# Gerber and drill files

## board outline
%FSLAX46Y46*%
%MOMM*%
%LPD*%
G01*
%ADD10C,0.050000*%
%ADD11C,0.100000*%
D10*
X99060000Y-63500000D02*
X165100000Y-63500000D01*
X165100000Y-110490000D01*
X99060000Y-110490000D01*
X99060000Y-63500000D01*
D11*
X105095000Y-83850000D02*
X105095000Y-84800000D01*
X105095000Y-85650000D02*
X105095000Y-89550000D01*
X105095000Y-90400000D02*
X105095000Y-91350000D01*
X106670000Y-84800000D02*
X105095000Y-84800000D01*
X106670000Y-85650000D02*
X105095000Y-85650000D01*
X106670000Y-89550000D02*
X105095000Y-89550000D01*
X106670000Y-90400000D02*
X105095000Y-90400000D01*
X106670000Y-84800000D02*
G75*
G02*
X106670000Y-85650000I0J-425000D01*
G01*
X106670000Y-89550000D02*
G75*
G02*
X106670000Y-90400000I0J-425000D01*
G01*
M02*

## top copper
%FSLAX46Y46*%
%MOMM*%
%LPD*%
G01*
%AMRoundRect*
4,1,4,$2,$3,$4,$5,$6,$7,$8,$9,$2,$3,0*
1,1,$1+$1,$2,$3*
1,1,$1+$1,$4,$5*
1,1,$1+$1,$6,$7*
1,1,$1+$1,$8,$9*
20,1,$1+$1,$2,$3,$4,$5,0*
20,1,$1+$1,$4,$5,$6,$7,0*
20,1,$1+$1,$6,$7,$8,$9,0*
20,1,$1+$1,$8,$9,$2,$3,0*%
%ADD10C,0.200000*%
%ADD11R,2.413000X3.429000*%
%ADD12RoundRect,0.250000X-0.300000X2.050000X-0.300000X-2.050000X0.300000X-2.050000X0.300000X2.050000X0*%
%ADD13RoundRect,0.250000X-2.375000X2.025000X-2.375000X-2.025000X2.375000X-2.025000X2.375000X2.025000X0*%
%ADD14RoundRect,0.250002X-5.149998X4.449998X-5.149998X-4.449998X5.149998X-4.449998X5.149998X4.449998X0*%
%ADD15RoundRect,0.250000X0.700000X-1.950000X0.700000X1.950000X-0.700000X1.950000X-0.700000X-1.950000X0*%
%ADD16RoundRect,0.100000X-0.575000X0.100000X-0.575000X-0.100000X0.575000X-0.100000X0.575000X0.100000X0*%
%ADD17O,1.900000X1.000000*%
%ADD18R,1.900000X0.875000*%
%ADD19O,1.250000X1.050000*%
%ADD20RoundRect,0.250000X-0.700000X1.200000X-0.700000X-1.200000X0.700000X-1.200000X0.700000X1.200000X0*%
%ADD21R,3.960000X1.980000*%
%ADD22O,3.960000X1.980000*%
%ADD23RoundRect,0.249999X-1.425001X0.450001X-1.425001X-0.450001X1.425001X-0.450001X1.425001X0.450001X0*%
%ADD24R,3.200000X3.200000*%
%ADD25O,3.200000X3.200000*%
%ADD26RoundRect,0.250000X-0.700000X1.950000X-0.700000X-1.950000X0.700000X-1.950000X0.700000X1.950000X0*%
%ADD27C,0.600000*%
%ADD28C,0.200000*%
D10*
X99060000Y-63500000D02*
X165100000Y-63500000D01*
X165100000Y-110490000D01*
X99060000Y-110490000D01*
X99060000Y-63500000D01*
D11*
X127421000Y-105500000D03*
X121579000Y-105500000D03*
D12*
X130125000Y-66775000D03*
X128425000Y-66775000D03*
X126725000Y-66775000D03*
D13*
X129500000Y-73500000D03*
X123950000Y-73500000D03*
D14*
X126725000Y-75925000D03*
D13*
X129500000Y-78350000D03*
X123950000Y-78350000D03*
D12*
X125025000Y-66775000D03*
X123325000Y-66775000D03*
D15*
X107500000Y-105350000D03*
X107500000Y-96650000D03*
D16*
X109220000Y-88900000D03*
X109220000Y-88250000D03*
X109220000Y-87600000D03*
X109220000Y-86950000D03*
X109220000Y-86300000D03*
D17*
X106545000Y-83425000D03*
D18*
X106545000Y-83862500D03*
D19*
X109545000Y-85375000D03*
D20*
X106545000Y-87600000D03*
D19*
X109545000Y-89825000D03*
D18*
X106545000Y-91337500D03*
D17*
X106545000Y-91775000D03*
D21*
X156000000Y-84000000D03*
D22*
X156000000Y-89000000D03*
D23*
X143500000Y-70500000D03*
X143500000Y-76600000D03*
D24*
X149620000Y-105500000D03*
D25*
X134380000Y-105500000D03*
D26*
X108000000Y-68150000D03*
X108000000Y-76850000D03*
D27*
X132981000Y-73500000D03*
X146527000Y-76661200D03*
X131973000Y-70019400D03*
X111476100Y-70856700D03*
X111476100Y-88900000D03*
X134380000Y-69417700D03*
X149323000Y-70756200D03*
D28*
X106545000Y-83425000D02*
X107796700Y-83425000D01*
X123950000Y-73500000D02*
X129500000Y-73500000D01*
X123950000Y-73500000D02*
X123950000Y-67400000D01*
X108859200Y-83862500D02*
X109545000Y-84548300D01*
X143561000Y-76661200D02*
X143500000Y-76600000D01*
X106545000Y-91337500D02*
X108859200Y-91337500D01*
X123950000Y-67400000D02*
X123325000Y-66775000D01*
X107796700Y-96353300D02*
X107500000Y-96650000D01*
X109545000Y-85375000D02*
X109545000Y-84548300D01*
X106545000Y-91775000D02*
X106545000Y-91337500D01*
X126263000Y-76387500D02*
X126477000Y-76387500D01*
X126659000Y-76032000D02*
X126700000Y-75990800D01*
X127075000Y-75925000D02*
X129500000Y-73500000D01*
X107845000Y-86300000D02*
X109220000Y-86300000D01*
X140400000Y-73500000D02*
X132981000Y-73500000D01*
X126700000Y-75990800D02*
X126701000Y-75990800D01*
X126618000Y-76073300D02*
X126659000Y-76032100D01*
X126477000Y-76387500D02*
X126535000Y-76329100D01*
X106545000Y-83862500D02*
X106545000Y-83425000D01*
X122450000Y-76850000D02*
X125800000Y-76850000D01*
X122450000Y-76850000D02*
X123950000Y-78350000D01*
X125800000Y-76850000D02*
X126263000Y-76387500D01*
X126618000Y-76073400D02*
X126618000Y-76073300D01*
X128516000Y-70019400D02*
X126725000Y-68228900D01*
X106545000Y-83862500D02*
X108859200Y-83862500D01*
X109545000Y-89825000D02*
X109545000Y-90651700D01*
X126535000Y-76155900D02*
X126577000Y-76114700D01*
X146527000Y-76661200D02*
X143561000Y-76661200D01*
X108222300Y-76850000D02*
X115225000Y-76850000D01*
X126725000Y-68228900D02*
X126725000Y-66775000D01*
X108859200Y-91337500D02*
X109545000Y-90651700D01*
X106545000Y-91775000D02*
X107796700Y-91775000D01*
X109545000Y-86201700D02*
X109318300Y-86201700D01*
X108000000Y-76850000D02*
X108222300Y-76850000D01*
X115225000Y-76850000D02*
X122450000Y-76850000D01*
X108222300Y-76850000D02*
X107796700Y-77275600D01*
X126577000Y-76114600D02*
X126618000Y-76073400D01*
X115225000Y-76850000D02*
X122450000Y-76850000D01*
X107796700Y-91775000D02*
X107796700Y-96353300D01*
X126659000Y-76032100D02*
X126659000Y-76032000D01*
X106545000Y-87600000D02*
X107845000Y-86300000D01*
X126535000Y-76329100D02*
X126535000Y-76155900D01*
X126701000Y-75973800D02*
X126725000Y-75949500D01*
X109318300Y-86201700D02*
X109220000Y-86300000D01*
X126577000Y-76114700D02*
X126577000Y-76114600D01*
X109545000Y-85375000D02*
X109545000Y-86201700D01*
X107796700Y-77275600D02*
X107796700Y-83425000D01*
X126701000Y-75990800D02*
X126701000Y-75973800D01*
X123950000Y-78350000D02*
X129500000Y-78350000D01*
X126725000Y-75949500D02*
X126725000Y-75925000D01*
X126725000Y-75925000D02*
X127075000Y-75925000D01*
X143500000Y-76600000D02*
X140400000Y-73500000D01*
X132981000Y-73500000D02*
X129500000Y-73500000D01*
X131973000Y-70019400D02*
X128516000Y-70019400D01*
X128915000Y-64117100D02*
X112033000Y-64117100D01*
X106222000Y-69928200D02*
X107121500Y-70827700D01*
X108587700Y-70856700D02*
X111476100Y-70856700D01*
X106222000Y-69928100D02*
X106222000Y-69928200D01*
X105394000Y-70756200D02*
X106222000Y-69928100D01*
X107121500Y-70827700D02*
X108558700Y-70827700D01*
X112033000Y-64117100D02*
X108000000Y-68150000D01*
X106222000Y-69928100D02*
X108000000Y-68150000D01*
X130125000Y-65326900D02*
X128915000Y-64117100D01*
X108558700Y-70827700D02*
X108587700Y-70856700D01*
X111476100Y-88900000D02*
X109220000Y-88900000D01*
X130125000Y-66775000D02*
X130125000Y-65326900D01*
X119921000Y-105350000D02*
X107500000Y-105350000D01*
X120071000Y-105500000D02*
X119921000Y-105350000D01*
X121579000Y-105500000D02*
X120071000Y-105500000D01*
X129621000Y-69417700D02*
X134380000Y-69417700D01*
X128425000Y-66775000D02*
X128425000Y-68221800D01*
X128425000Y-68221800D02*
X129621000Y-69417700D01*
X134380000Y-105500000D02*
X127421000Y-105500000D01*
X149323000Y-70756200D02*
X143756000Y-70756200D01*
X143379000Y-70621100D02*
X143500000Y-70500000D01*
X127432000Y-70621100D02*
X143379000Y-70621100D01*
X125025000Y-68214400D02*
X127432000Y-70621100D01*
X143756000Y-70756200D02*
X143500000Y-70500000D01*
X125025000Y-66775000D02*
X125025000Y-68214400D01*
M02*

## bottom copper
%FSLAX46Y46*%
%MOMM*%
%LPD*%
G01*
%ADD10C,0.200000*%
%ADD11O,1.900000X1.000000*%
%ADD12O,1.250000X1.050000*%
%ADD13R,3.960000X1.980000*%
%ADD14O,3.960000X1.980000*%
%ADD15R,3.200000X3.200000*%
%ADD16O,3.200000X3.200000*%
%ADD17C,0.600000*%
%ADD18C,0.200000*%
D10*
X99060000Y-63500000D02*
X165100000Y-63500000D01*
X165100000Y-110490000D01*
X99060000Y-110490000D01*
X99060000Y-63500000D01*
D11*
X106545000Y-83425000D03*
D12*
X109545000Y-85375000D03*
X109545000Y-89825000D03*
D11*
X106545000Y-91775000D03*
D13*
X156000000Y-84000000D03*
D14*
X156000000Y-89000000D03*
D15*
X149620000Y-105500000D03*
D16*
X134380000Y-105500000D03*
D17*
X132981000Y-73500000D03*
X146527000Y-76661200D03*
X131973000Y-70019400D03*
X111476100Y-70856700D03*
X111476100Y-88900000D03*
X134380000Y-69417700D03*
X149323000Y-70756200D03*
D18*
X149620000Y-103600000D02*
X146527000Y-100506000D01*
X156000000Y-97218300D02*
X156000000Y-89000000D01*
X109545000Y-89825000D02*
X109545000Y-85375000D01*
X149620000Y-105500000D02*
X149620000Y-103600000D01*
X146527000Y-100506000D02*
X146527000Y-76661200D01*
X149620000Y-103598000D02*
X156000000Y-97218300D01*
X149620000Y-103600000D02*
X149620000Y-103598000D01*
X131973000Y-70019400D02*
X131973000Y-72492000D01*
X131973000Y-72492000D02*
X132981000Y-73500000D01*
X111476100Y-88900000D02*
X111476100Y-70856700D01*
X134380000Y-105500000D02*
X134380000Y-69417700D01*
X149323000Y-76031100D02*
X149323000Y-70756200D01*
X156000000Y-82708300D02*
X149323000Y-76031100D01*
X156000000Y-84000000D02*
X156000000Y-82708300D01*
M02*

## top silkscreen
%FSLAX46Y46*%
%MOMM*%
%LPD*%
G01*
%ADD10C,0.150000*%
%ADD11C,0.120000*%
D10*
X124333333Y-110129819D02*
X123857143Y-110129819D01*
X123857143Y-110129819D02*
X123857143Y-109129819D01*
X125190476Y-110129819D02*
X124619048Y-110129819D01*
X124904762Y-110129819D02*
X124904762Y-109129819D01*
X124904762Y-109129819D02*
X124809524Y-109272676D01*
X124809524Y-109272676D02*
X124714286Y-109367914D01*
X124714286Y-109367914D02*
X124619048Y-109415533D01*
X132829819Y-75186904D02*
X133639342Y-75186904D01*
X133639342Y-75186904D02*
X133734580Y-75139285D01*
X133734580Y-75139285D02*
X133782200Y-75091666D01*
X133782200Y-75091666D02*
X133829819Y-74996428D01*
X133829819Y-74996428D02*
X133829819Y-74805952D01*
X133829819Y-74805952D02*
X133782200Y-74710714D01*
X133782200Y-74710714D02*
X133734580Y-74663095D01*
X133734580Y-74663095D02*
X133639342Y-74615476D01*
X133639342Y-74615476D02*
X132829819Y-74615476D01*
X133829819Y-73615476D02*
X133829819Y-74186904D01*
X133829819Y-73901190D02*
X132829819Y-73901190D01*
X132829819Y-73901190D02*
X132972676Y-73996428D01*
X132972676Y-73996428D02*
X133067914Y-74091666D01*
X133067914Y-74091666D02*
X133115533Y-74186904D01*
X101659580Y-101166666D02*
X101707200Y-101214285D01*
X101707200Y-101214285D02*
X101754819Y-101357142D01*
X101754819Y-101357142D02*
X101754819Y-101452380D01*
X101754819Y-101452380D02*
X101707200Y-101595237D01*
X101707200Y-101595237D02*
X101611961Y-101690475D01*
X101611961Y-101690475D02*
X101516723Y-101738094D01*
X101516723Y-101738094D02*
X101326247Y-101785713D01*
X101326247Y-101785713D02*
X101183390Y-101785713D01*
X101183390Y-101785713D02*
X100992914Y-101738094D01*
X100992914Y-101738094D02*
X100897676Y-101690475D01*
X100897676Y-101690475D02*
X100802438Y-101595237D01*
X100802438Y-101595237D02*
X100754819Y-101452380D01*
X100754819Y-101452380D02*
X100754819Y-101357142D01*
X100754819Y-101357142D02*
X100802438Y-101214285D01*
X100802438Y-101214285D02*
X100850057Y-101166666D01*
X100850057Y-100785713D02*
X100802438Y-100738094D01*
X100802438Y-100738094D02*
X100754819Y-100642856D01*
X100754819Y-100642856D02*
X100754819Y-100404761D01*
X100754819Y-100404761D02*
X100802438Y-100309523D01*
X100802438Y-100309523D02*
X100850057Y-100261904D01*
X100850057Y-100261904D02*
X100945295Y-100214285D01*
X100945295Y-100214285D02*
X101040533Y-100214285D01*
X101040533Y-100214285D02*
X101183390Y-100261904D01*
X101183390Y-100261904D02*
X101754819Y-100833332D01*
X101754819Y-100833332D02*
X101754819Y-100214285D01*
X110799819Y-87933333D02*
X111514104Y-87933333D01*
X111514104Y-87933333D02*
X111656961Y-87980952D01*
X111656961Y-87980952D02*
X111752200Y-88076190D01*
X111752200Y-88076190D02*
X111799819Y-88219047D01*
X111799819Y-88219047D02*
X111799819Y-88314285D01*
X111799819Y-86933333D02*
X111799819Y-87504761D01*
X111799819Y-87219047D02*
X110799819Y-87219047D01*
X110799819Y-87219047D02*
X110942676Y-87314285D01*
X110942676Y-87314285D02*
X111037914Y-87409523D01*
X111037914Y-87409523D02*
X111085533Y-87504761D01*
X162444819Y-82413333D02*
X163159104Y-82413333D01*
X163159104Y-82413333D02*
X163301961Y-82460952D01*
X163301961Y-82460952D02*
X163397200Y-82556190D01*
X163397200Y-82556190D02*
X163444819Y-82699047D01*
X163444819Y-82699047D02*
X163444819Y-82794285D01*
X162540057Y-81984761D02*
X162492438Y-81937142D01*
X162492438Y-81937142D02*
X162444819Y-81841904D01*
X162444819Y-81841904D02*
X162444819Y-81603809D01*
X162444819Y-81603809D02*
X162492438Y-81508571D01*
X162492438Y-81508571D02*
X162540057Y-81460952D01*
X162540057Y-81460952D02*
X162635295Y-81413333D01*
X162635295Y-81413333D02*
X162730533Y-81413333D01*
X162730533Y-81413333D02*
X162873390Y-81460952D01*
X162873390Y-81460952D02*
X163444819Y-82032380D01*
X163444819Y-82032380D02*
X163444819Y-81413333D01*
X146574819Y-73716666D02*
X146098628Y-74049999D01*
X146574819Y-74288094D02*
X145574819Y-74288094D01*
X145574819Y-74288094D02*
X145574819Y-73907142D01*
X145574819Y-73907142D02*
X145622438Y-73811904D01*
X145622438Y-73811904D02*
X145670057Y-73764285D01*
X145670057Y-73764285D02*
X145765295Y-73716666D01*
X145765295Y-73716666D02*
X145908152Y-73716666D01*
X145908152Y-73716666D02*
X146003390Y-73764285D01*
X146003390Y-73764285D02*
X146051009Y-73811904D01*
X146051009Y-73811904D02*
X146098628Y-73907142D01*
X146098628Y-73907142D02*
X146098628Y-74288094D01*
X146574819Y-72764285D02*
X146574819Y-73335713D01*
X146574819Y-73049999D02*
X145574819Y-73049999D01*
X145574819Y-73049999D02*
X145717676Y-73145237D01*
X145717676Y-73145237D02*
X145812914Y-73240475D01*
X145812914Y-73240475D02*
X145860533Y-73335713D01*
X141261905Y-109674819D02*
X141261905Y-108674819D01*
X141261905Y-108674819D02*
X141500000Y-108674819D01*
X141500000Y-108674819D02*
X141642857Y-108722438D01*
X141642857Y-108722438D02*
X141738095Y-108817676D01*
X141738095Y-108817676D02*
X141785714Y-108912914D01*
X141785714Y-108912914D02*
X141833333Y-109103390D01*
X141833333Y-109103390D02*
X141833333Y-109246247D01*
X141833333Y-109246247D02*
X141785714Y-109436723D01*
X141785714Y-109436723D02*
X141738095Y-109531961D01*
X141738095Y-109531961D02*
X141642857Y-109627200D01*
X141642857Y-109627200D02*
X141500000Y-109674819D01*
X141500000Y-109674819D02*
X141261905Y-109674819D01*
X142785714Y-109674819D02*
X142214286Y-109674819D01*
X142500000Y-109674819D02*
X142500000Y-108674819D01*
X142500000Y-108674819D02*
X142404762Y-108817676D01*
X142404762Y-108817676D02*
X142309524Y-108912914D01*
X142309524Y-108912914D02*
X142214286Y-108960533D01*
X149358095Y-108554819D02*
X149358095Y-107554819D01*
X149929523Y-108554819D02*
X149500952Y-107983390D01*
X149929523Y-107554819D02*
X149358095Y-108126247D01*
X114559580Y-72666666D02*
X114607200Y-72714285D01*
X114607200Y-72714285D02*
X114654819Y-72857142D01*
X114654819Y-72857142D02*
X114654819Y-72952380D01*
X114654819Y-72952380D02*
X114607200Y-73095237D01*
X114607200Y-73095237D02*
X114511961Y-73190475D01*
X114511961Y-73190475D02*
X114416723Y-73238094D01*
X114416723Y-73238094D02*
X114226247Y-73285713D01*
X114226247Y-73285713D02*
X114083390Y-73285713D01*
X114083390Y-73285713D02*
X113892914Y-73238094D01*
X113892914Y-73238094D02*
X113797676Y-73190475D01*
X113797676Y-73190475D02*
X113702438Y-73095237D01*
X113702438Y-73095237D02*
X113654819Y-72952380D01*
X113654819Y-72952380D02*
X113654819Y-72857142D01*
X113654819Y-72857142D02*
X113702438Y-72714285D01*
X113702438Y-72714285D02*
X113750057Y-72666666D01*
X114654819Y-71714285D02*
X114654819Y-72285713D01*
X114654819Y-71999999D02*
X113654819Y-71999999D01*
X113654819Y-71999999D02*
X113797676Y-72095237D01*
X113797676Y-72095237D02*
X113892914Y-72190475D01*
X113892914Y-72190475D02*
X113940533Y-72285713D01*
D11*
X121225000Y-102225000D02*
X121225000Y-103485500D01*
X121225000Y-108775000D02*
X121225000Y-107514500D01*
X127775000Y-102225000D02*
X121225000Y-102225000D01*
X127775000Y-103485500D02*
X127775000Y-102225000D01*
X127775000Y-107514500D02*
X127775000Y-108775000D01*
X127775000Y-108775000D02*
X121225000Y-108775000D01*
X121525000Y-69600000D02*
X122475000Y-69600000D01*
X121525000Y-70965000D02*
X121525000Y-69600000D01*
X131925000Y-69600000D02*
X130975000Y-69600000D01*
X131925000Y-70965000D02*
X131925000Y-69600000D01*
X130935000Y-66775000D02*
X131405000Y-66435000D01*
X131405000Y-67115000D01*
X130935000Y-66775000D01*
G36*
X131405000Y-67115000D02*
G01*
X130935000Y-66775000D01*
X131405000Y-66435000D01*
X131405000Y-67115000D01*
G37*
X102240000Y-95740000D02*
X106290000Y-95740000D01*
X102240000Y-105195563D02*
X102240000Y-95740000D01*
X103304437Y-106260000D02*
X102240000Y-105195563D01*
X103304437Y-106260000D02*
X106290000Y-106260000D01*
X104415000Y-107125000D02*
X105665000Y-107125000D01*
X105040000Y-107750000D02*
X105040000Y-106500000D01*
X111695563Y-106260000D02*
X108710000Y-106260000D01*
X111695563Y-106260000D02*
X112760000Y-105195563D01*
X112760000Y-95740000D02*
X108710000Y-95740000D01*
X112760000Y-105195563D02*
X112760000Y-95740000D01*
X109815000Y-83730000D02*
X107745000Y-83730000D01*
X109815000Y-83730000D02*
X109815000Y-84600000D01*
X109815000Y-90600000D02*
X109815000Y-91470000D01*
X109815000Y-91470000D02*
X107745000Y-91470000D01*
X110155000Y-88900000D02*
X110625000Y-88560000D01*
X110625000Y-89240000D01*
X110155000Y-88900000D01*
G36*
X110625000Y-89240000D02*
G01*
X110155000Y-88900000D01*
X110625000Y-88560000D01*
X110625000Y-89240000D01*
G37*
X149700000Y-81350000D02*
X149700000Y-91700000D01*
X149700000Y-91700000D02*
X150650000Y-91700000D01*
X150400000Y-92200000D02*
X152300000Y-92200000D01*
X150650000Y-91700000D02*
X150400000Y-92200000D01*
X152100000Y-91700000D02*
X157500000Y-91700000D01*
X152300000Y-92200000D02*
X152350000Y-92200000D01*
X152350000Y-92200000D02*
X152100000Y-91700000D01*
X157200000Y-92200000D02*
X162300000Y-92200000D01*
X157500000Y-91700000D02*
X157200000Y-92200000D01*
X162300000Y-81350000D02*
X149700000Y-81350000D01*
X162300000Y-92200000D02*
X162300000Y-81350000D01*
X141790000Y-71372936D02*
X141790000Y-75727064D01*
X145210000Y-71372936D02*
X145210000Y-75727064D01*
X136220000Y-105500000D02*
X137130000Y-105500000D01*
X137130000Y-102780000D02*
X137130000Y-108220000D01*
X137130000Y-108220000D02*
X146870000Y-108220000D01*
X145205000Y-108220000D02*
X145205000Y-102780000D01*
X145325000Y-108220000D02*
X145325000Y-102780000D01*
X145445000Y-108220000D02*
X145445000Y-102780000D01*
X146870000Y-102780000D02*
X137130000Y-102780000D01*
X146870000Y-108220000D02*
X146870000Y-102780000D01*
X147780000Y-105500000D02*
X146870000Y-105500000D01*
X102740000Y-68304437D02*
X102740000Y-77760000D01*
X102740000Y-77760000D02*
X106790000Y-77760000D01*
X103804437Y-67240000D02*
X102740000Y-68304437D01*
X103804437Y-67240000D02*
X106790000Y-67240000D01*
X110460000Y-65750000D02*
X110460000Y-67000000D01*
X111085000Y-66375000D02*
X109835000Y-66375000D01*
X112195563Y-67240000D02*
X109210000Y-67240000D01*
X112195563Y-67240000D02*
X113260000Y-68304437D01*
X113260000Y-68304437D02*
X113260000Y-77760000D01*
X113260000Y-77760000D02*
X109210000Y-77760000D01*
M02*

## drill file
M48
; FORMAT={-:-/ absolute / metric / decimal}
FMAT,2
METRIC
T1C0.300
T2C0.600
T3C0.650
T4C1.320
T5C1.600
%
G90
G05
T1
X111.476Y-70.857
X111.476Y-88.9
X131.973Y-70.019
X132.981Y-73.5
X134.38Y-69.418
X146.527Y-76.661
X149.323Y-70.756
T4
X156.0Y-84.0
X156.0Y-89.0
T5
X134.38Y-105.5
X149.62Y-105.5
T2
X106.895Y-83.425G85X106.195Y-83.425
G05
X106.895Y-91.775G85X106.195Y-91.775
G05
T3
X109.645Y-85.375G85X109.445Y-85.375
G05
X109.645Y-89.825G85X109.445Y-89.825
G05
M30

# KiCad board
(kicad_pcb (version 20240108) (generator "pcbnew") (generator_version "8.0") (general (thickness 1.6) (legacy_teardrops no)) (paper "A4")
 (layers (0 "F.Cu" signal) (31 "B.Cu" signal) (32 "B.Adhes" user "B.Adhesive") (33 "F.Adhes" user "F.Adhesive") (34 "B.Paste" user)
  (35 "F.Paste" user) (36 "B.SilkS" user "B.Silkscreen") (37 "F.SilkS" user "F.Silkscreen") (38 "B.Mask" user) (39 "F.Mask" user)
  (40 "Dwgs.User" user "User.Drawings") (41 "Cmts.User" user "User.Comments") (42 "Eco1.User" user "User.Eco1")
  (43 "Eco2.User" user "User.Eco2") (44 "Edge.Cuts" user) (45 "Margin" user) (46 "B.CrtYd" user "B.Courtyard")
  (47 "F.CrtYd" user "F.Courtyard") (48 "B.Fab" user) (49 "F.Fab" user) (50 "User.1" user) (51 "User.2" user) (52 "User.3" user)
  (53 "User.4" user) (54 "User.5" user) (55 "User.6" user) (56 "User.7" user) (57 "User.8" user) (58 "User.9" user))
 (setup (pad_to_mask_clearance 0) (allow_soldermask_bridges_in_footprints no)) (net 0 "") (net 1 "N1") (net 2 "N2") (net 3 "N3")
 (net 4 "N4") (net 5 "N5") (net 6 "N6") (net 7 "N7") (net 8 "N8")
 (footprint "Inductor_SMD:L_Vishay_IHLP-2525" (layer "F.Cu") (at 124.5 105.5 180)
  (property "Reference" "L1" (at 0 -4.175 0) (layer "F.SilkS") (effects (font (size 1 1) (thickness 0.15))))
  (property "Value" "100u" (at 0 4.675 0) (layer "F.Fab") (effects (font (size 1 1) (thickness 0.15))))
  (fp_line (start 3.275 3.275) (end 3.275 2.0145) (stroke (width 0.12) (type solid)) (layer "F.SilkS"))
  (fp_line (start 3.275 -3.275) (end 3.275 -2.0145) (stroke (width 0.12) (type solid)) (layer "F.SilkS"))
  (fp_line (start -3.275 3.275) (end 3.275 3.275) (stroke (width 0.12) (type solid)) (layer "F.SilkS"))
  (fp_line (start -3.275 2.0145) (end -3.275 3.275) (stroke (width 0.12) (type solid)) (layer "F.SilkS"))
  (fp_line (start -3.275 -2.0145) (end -3.275 -3.275) (stroke (width 0.12) (type solid)) (layer "F.SilkS"))
  (fp_line (start -3.275 -3.275) (end 3.275 -3.275) (stroke (width 0.12) (type solid)) (layer "F.SilkS"))
  (pad "1" smd rect (at -2.921 0 180) (size 2.413 3.429) (layers "F.Cu" "F.Paste" "F.Mask") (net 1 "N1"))
  (pad "2" smd rect (at 2.921 0 180) (size 2.413 3.429) (layers "F.Cu" "F.Paste" "F.Mask") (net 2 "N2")))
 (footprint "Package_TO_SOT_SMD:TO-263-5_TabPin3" (layer "F.Cu") (at 126.725 74.425 -90)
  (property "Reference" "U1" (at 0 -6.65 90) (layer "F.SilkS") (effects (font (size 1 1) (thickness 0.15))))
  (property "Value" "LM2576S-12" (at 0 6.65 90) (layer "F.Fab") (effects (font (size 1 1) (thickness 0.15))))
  (fp_line (start -4.825 5.2) (end -4.825 4.25) (stroke (width 0.12) (type solid)) (layer "F.SilkS"))
  (fp_line (start -3.46 5.2) (end -4.825 5.2) (stroke (width 0.12) (type solid)) (layer "F.SilkS"))
  (fp_line (start -4.825 -5.2) (end -4.825 -4.25) (stroke (width 0.12) (type solid)) (layer "F.SilkS"))
  (fp_line (start -3.46 -5.2) (end -4.825 -5.2) (stroke (width 0.12) (type solid)) (layer "F.SilkS"))
  (fp_poly
   (pts (xy -7.65 -4.21) (xy -7.99 -4.68) (xy -7.31 -4.68) (xy -7.65 -4.21)) (stroke (width 0.12) (type solid)) (fill solid)
   (layer "F.SilkS"))
  (pad "1" smd roundrect (at -7.65 -3.4 270) (size 4.6 1.1) (layers "F.Cu" "F.Paste" "F.Mask") (roundrect_rratio 0.227273) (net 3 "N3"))
  (pad "2" smd roundrect (at -7.65 -1.7 270) (size 4.6 1.1) (layers "F.Cu" "F.Paste" "F.Mask") (roundrect_rratio 0.227273) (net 1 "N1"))
  (pad "3" smd roundrect (at -7.65 0 270) (size 4.6 1.1) (layers "F.Cu" "F.Paste" "F.Mask") (roundrect_rratio 0.227273) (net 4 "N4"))
  (pad "3" smd roundrect (at -0.925 -2.775 270) (size 4.55 5.25) (layers "F.Cu" "F.Paste") (roundrect_rratio 0.054945) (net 4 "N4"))
  (pad "3" smd roundrect (at -0.925 2.775 270) (size 4.55 5.25) (layers "F.Cu" "F.Paste") (roundrect_rratio 0.054945) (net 4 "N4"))
  (pad "3" smd roundrect (at 1.5 0 270) (size 9.4 10.8) (layers "F.Cu" "F.Mask") (roundrect_rratio 0.026596) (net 4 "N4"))
  (pad "3" smd roundrect (at 3.925 -2.775 270) (size 4.55 5.25) (layers "F.Cu" "F.Paste") (roundrect_rratio 0.054945) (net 4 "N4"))
  (pad "3" smd roundrect (at 3.925 2.775 270) (size 4.55 5.25) (layers "F.Cu" "F.Paste") (roundrect_rratio 0.054945) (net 4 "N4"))
  (pad "4" smd roundrect (at -7.65 1.7 270) (size 4.6 1.1) (layers "F.Cu" "F.Paste" "F.Mask") (roundrect_rratio 0.227273) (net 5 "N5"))
  (pad "5" smd roundrect (at -7.65 3.4 270) (size 4.6 1.1) (layers "F.Cu" "F.Paste" "F.Mask") (roundrect_rratio 0.227273) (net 4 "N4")))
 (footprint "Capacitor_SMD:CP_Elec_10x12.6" (layer "F.Cu") (at 107.5 101 90)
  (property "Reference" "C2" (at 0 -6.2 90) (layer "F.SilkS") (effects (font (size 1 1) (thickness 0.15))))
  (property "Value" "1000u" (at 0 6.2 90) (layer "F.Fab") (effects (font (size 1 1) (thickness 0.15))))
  (fp_line (start 5.26 -5.26) (end 5.26 -1.21) (stroke (width 0.12) (type solid)) (layer "F.SilkS"))
  (fp_line (start -4.195563 -5.26) (end 5.26 -5.26) (stroke (width 0.12) (type solid)) (layer "F.SilkS"))
  (fp_line (start -5.26 -4.195563) (end -4.195563 -5.26) (stroke (width 0.12) (type solid)) (layer "F.SilkS"))
  (fp_line (start -5.26 -4.195563) (end -5.26 -1.21) (stroke (width 0.12) (type solid)) (layer "F.SilkS"))
  (fp_line (start -6.125 -3.085) (end -6.125 -1.835) (stroke (width 0.12) (type solid)) (layer "F.SilkS"))
  (fp_line (start -6.75 -2.46) (end -5.5 -2.46) (stroke (width 0.12) (type solid)) (layer "F.SilkS"))
  (fp_line (start -5.26 4.195563) (end -5.26 1.21) (stroke (width 0.12) (type solid)) (layer "F.SilkS"))
  (fp_line (start -5.26 4.195563) (end -4.195563 5.26) (stroke (width 0.12) (type solid)) (layer "F.SilkS"))
  (fp_line (start 5.26 5.26) (end 5.26 1.21) (stroke (width 0.12) (type solid)) (layer "F.SilkS"))
  (fp_line (start -4.195563 5.26) (end 5.26 5.26) (stroke (width 0.12) (type solid)) (layer "F.SilkS"))
  (pad "1" smd roundrect (at -4.35 0 90) (size 4.4 1.9) (layers "F.Cu" "F.Paste" "F.Mask") (roundrect_rratio 0.131579) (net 2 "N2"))
  (pad "2" smd roundrect (at 4.35 0 90) (size 4.4 1.9) (layers "F.Cu" "F.Paste" "F.Mask") (roundrect_rratio 0.131579) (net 4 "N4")))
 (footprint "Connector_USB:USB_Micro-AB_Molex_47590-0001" (layer "F.Cu") (at 106.195 87.6 -90)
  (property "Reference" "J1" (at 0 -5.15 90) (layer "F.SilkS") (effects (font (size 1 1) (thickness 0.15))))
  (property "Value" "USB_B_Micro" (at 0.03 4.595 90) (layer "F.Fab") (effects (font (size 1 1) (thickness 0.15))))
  (fp_line (start -3.87 -3.62) (end -3.87 -1.55) (stroke (width 0.12) (type solid)) (layer "F.SilkS"))
  (fp_line (start -3.87 -3.62) (end -3 -3.62) (stroke (width 0.12) (type solid)) (layer "F.SilkS"))
  (fp_line (start 3 -3.62) (end 3.87 -3.62) (stroke (width 0.12) (type solid)) (layer "F.SilkS"))
  (fp_line (start 3.87 -3.62) (end 3.87 -1.55) (stroke (width 0.12) (type solid)) (layer "F.SilkS"))
  (fp_poly
   (pts (xy 1.3 -3.96) (xy 0.96 -4.43) (xy 1.64 -4.43) (xy 1.3 -3.96)) (stroke (width 0.12) (type solid)) (fill solid) (layer "F.SilkS"))
  (fp_line (start -3.75 1.1) (end -2.8 1.1) (stroke (width 0.1) (type solid)) (layer "Edge.Cuts"))
  (fp_line (start -1.95 1.1) (end 1.95 1.1) (stroke (width 0.1) (type solid)) (layer "Edge.Cuts"))
  (fp_line (start 2.8 1.1) (end 3.75 1.1) (stroke (width 0.1) (type solid)) (layer "Edge.Cuts"))
  (fp_line (start -2.8 -0.475) (end -2.8 1.1) (stroke (width 0.1) (type solid)) (layer "Edge.Cuts"))
  (fp_line (start -1.95 -0.475) (end -1.95 1.1) (stroke (width 0.1) (type solid)) (layer "Edge.Cuts"))
  (fp_line (start 1.95 -0.475) (end 1.95 1.1) (stroke (width 0.1) (type solid)) (layer "Edge.Cuts"))
  (fp_line (start 2.8 -0.475) (end 2.8 1.1) (stroke (width 0.1) (type solid)) (layer "Edge.Cuts"))
  (fp_arc (start -2.8 -0.475) (mid -2.375 -0.9) (end -1.95 -0.475) (stroke (width 0.1) (type solid)) (layer "Edge.Cuts"))
  (fp_arc (start 1.95 -0.475) (mid 2.375 -0.9) (end 2.8 -0.475) (stroke (width 0.1) (type solid)) (layer "Edge.Cuts"))
  (pad "" smd rect (at -3.5 -0.35 270) (size 0.3 0.85) (layers "F.Paste"))
  (pad "" smd rect (at 3.5 -0.35 270) (size 0.3 0.85) (layers "F.Paste"))
  (pad "1" smd roundrect (at 1.3 -3.025 270) (size 0.4 1.35) (layers "F.Cu" "F.Paste" "F.Mask") (roundrect_rratio 0.25) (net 3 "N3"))
  (pad "2" smd roundrect (at 0.65 -3.025 270) (size 0.4 1.35) (layers "F.Cu" "F.Paste" "F.Mask") (roundrect_rratio 0.25) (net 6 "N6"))
  (pad "3" smd roundrect (at 0 -3.025 270) (size 0.4 1.35) (layers "F.Cu" "F.Paste" "F.Mask") (roundrect_rratio 0.25) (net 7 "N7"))
  (pad "4" smd roundrect (at -0.65 -3.025 270) (size 0.4 1.35) (layers "F.Cu" "F.Paste" "F.Mask") (roundrect_rratio 0.25) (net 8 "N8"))
  (pad "5" smd roundrect (at -1.3 -3.025 270) (size 0.4 1.35) (layers "F.Cu" "F.Paste" "F.Mask") (roundrect_rratio 0.25) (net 4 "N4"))
  (pad "6" thru_hole oval (at -4.175 -0.35 270) (size 1 1.9) (drill oval 0.6 1.3) (layers "*.Cu" "*.Mask") (remove_unused_layers no)
   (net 4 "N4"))
  (pad "6" smd rect (at -3.7375 -0.35 270) (size 0.875 1.9) (layers "F.Cu" "F.Mask") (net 4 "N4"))
  (pad "6" thru_hole oval (at -2.225 -3.35 270) (size 1.05 1.25) (drill oval 0.65 0.85) (layers "*.Cu" "*.Mask") (remove_unused_layers no)
   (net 4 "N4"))
  (pad "6" smd roundrect (at 0 -0.35 270) (size 2.9 1.9) (layers "F.Cu" "F.Paste" "F.Mask") (roundrect_rratio 0.1315789474) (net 4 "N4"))
  (pad "6" thru_hole oval (at 2.225 -3.35 270) (size 1.05 1.25) (drill oval 0.65 0.85) (layers "*.Cu" "*.Mask") (remove_unused_layers no)
   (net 4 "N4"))
  (pad "6" smd rect (at 3.7375 -0.35 270) (size 0.875 1.9) (layers "F.Cu" "F.Mask") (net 4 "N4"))
  (pad "6" thru_hole oval (at 4.175 -0.35 270) (size 1 1.9) (drill oval 0.6 1.3) (layers "*.Cu" "*.Mask") (remove_unused_layers no)
   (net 4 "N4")))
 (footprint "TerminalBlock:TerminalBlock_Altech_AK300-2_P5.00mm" (layer "F.Cu") (at 156 84 -90)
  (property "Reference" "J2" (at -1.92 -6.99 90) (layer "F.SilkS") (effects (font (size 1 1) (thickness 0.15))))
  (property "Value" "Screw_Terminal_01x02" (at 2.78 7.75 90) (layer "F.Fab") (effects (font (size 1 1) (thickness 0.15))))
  (fp_line (start -2.65 6.3) (end 7.7 6.3) (stroke (width 0.12) (type solid)) (layer "F.SilkS"))
  (fp_line (start 7.7 6.3) (end 7.7 5.35) (stroke (width 0.12) (type solid)) (layer "F.SilkS"))
  (fp_line (start 8.2 5.6) (end 8.2 3.7) (stroke (width 0.12) (type solid)) (layer "F.SilkS"))
  (fp_line (start 7.7 5.35) (end 8.2 5.6) (stroke (width 0.12) (type solid)) (layer "F.SilkS"))
  (fp_line (start 7.7 3.9) (end 7.7 -1.5) (stroke (width 0.12) (type solid)) (layer "F.SilkS"))
  (fp_line (start 8.2 3.7) (end 8.2 3.65) (stroke (width 0.12) (type solid)) (layer "F.SilkS"))
  (fp_line (start 8.2 3.65) (end 7.7 3.9) (stroke (width 0.12) (type solid)) (layer "F.SilkS"))
  (fp_line (start 8.2 -1.2) (end 8.2 -6.3) (stroke (width 0.12) (type solid)) (layer "F.SilkS"))
  (fp_line (start 7.7 -1.5) (end 8.2 -1.2) (stroke (width 0.12) (type solid)) (layer "F.SilkS"))
  (fp_line (start -2.65 -6.3) (end -2.65 6.3) (stroke (width 0.12) (type solid)) (layer "F.SilkS"))
  (fp_line (start 8.2 -6.3) (end -2.65 -6.3) (stroke (width 0.12) (type solid)) (layer "F.SilkS"))
  (pad "1" thru_hole rect (at 0 0 270) (size 1.98 3.96) (drill 1.32) (layers "*.Cu" "*.Mask") (remove_unused_layers no) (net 5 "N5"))
  (pad "2" thru_hole oval (at 5 0 270) (size 1.98 3.96) (drill 1.32) (layers "*.Cu" "*.Mask") (remove_unused_layers no) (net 4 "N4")))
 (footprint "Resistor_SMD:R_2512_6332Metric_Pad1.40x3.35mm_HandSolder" (layer "F.Cu") (at 143.5 73.55 -90)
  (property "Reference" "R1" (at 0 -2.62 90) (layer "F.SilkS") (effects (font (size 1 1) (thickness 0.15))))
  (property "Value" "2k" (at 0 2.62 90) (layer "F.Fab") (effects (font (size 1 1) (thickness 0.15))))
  (fp_line (start -2.177064 1.71) (end 2.177064 1.71) (stroke (width 0.12) (type solid)) (layer "F.SilkS"))
  (fp_line (start -2.177064 -1.71) (end 2.177064 -1.71) (stroke (width 0.12) (type solid)) (layer "F.SilkS"))
  (pad "1" smd roundrect (at -3.05 0 270) (size 1.4 3.35) (layers "F.Cu" "F.Paste" "F.Mask") (roundrect_rratio 0.178571) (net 5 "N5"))
  (pad "2" smd roundrect (at 3.05 0 270) (size 1.4 3.35) (layers "F.Cu" "F.Paste" "F.Mask") (roundrect_rratio 0.178571) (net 4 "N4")))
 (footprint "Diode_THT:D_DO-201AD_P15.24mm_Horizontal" (layer "F.Cu") (at 149.62 105.5 180)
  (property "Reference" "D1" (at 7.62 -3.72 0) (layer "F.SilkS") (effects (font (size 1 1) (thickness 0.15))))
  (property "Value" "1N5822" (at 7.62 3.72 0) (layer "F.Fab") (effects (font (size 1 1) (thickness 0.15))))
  (fp_line (start 13.4 0) (end 12.49 0) (stroke (width 0.12) (type solid)) (layer "F.SilkS"))
  (fp_line (start 12.49 2.72) (end 12.49 -2.72) (stroke (width 0.12) (type solid)) (layer "F.SilkS"))
  (fp_line (start 12.49 -2.72) (end 2.75 -2.72) (stroke (width 0.12) (type solid)) (layer "F.SilkS"))
  (fp_line (start 4.415 -2.72) (end 4.415 2.72) (stroke (width 0.12) (type solid)) (layer "F.SilkS"))
  (fp_line (start 4.295 -2.72) (end 4.295 2.72) (stroke (width 0.12) (type solid)) (layer "F.SilkS"))
  (fp_line (start 4.175 -2.72) (end 4.175 2.72) (stroke (width 0.12) (type solid)) (layer "F.SilkS"))
  (fp_line (start 2.75 2.72) (end 12.49 2.72) (stroke (width 0.12) (type solid)) (layer "F.SilkS"))
  (fp_line (start 2.75 -2.72) (end 2.75 2.72) (stroke (width 0.12) (type solid)) (layer "F.SilkS"))
  (fp_line (start 1.84 0) (end 2.75 0) (stroke (width 0.12) (type solid)) (layer "F.SilkS"))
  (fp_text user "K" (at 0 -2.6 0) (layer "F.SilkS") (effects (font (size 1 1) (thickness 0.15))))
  (pad "1" thru_hole rect (at 0 0 180) (size 3.2 3.2) (drill 1.6) (layers "*.Cu" "*.Mask") (remove_unused_layers no) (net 4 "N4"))
  (pad "2" thru_hole oval (at 15.24 0 180) (size 3.2 3.2) (drill 1.6) (layers "*.Cu" "*.Mask") (remove_unused_layers no) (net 1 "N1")))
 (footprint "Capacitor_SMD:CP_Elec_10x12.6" (layer "F.Cu") (at 108 72.5 -90)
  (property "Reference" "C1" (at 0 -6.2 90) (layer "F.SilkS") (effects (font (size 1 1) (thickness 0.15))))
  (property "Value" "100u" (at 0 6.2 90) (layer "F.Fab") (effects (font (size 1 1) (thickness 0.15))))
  (fp_line (start -4.195563 5.26) (end 5.26 5.26) (stroke (width 0.12) (type solid)) (layer "F.SilkS"))
  (fp_line (start 5.26 5.26) (end 5.26 1.21) (stroke (width 0.12) (type solid)) (layer "F.SilkS"))
  (fp_line (start -5.26 4.195563) (end -4.195563 5.26) (stroke (width 0.12) (type solid)) (layer "F.SilkS"))
  (fp_line (start -5.26 4.195563) (end -5.26 1.21) (stroke (width 0.12) (type solid)) (layer "F.SilkS"))
  (fp_line (start -6.75 -2.46) (end -5.5 -2.46) (stroke (width 0.12) (type solid)) (layer "F.SilkS"))
  (fp_line (start -6.125 -3.085) (end -6.125 -1.835) (stroke (width 0.12) (type solid)) (layer "F.SilkS"))
  (fp_line (start -5.26 -4.195563) (end -5.26 -1.21) (stroke (width 0.12) (type solid)) (layer "F.SilkS"))
  (fp_line (start -5.26 -4.195563) (end -4.195563 -5.26) (stroke (width 0.12) (type solid)) (layer "F.SilkS"))
  (fp_line (start -4.195563 -5.26) (end 5.26 -5.26) (stroke (width 0.12) (type solid)) (layer "F.SilkS"))
  (fp_line (start 5.26 -5.26) (end 5.26 -1.21) (stroke (width 0.12) (type solid)) (layer "F.SilkS"))
  (pad "1" smd roundrect (at -4.35 0 270) (size 4.4 1.9) (layers "F.Cu" "F.Paste" "F.Mask") (roundrect_rratio 0.131579) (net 3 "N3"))
  (pad "2" smd roundrect (at 4.35 0 270) (size 4.4 1.9) (layers "F.Cu" "F.Paste" "F.Mask") (roundrect_rratio 0.131579) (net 4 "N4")))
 (gr_rect (start 99.06 63.5) (end 165.1 110.49) (stroke (width 0.2) (type default)) (fill none) (layer "F.Cu"))
 (gr_rect (start 99.06 63.5) (end 165.1 110.49) (stroke (width 0.2) (type default)) (fill none) (layer "B.Cu"))
 (gr_rect (start 99.06 63.5) (end 165.1 110.49) (stroke (width 0.05) (type default)) (fill none) (layer "Edge.Cuts"))
 (segment (start 106.545 83.425) (end 107.7967 83.425) (width 0.2) (layer "F.Cu") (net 4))
 (segment (start 123.95 73.5) (end 129.5 73.5) (width 0.2) (layer "F.Cu") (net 4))
 (segment (start 123.95 73.5) (end 123.95 67.4) (width 0.2) (layer "F.Cu") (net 4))
 (segment (start 108.8592 83.8625) (end 109.545 84.5483) (width 0.2) (layer "F.Cu") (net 4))
 (segment (start 143.561 76.6612) (end 143.5 76.6) (width 0.2) (layer "F.Cu") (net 4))
 (segment (start 106.545 91.3375) (end 108.8592 91.3375) (width 0.2) (layer "F.Cu") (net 4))
 (segment (start 123.95 67.4) (end 123.325 66.775) (width 0.2) (layer "F.Cu") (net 4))
 (segment (start 107.7967 96.3533) (end 107.5 96.65) (width 0.2) (layer "F.Cu") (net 4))
 (segment (start 109.545 85.375) (end 109.545 84.5483) (width 0.2) (layer "F.Cu") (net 4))
 (segment (start 106.545 91.775) (end 106.545 91.3375) (width 0.2) (layer "F.Cu") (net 4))
 (segment (start 126.263 76.3875) (end 126.477 76.3875) (width 0.2) (layer "F.Cu") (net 4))
 (segment (start 126.659 76.032) (end 126.7 75.9908) (width 0.2) (layer "F.Cu") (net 4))
 (segment (start 127.075 75.925) (end 129.5 73.5) (width 0.2) (layer "F.Cu") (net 4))
 (segment (start 107.845 86.3) (end 109.22 86.3) (width 0.2) (layer "F.Cu") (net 4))
 (segment (start 140.4 73.5) (end 132.981 73.5) (width 0.2) (layer "F.Cu") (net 4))
 (segment (start 126.7 75.9908) (end 126.701 75.9908) (width 0.2) (layer "F.Cu") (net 4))
 (segment (start 126.618 76.0733) (end 126.659 76.0321) (width 0.2) (layer "F.Cu") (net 4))
 (segment (start 126.477 76.3875) (end 126.535 76.3291) (width 0.2) (layer "F.Cu") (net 4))
 (segment (start 106.545 83.8625) (end 106.545 83.425) (width 0.2) (layer "F.Cu") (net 4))
 (segment (start 122.45 76.85) (end 125.8 76.85) (width 0.2) (layer "F.Cu") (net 4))
 (segment (start 122.45 76.85) (end 123.95 78.35) (width 0.2) (layer "F.Cu") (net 4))
 (segment (start 125.8 76.85) (end 126.263 76.3875) (width 0.2) (layer "F.Cu") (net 4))
 (segment (start 126.618 76.0734) (end 126.618 76.0733) (width 0.2) (layer "F.Cu") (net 4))
 (segment (start 128.516 70.0194) (end 126.725 68.2289) (width 0.2) (layer "F.Cu") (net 4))
 (segment (start 106.545 83.8625) (end 108.8592 83.8625) (width 0.2) (layer "F.Cu") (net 4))
 (segment (start 109.545 89.825) (end 109.545 90.6517) (width 0.2) (layer "F.Cu") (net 4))
 (segment (start 126.535 76.1559) (end 126.577 76.1147) (width 0.2) (layer "F.Cu") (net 4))
 (segment (start 146.527 76.6612) (end 143.561 76.6612) (width 0.2) (layer "F.Cu") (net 4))
 (segment (start 108.2223 76.85) (end 115.225 76.85) (width 0.2) (layer "F.Cu") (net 4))
 (segment (start 126.725 68.2289) (end 126.725 66.775) (width 0.2) (layer "F.Cu") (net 4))
 (segment (start 108.8592 91.3375) (end 109.545 90.6517) (width 0.2) (layer "F.Cu") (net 4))
 (segment (start 106.545 91.775) (end 107.7967 91.775) (width 0.2) (layer "F.Cu") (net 4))
 (segment (start 109.545 86.2017) (end 109.3183 86.2017) (width 0.2) (layer "F.Cu") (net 4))
 (segment (start 108 76.85) (end 108.2223 76.85) (width 0.2) (layer "F.Cu") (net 4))
 (segment (start 115.225 76.85) (end 122.45 76.85) (width 0.2) (layer "F.Cu") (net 4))
 (segment (start 108.2223 76.85) (end 107.7967 77.2756) (width 0.2) (layer "F.Cu") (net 4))
 (segment (start 126.577 76.1146) (end 126.618 76.0734) (width 0.2) (layer "F.Cu") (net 4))
 (segment (start 115.225 76.85) (end 122.45 76.85) (width 0.2) (layer "F.Cu") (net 4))
 (segment (start 107.7967 91.775) (end 107.7967 96.3533) (width 0.2) (layer "F.Cu") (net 4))
 (segment (start 126.659 76.0321) (end 126.659 76.032) (width 0.2) (layer "F.Cu") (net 4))
 (segment (start 106.545 87.6) (end 107.845 86.3) (width 0.2) (layer "F.Cu") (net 4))
 (segment (start 126.535 76.3291) (end 126.535 76.1559) (width 0.2) (layer "F.Cu") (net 4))
 (segment (start 126.701 75.9738) (end 126.725 75.9495) (width 0.2) (layer "F.Cu") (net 4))
 (segment (start 109.3183 86.2017) (end 109.22 86.3) (width 0.2) (layer "F.Cu") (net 4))
 (segment (start 126.577 76.1147) (end 126.577 76.1146) (width 0.2) (layer "F.Cu") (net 4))
 (segment (start 109.545 85.375) (end 109.545 86.2017) (width 0.2) (layer "F.Cu") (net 4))
 (segment (start 107.7967 77.2756) (end 107.7967 83.425) (width 0.2) (layer "F.Cu") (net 4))
 (segment (start 126.701 75.9908) (end 126.701 75.9738) (width 0.2) (layer "F.Cu") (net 4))
 (segment (start 123.95 78.35) (end 129.5 78.35) (width 0.2) (layer "F.Cu") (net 4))
 (segment (start 126.725 75.9495) (end 126.725 75.925) (width 0.2) (layer "F.Cu") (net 4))
 (segment (start 126.725 75.925) (end 127.075 75.925) (width 0.2) (layer "F.Cu") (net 4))
 (segment (start 143.5 76.6) (end 140.4 73.5) (width 0.2) (layer "F.Cu") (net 4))
 (segment (start 132.981 73.5) (end 129.5 73.5) (width 0.2) (layer "F.Cu") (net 4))
 (segment (start 131.973 70.0194) (end 128.516 70.0194) (width 0.2) (layer "F.Cu") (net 4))
 (via (at 132.981 73.5) (size 0.6) (drill 0.3) (layers "F.Cu" "B.Cu") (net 4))
 (via (at 146.527 76.6612) (size 0.6) (drill 0.3) (layers "F.Cu" "B.Cu") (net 4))
 (via (at 131.973 70.0194) (size 0.6) (drill 0.3) (layers "F.Cu" "B.Cu") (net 4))
 (segment (start 149.62 103.6) (end 146.527 100.506) (width 0.2) (layer "B.Cu") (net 4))
 (segment (start 156 97.2183) (end 156 89) (width 0.2) (layer "B.Cu") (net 4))
 (segment (start 109.545 89.825) (end 109.545 85.375) (width 0.2) (layer "B.Cu") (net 4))
 (segment (start 149.62 105.5) (end 149.62 103.6) (width 0.2) (layer "B.Cu") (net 4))
 (segment (start 146.527 100.506) (end 146.527 76.6612) (width 0.2) (layer "B.Cu") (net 4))
 (segment (start 149.62 103.598) (end 156 97.2183) (width 0.2) (layer "B.Cu") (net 4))
 (segment (start 149.62 103.6) (end 149.62 103.598) (width 0.2) (layer "B.Cu") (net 4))
 (segment (start 131.973 70.0194) (end 131.973 72.492) (width 0.2) (layer "B.Cu") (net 4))
 (segment (start 131.973 72.492) (end 132.981 73.5) (width 0.2) (layer "B.Cu") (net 4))
 (segment (start 128.915 64.1171) (end 112.033 64.1171) (width 0.2) (layer "F.Cu") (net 3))
 (segment (start 106.222 69.9282) (end 107.1215 70.8277) (width 0.2) (layer "F.Cu") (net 3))
 (segment (start 108.5877 70.8567) (end 111.4761 70.8567) (width 0.2) (layer "F.Cu") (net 3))
 (segment (start 106.222 69.9281) (end 106.222 69.9282) (width 0.2) (layer "F.Cu") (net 3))
 (segment (start 105.394 70.7562) (end 106.222 69.9281) (width 0.2) (layer "F.Cu") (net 3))
 (segment (start 107.1215 70.8277) (end 108.5587 70.8277) (width 0.2) (layer "F.Cu") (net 3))
 (segment (start 112.033 64.1171) (end 108 68.15) (width 0.2) (layer "F.Cu") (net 3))
 (segment (start 106.222 69.9281) (end 108 68.15) (width 0.2) (layer "F.Cu") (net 3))
 (segment (start 130.125 65.3269) (end 128.915 64.1171) (width 0.2) (layer "F.Cu") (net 3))
 (segment (start 108.5587 70.8277) (end 108.5877 70.8567) (width 0.2) (layer "F.Cu") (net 3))
 (segment (start 111.4761 88.9) (end 109.22 88.9) (width 0.2) (layer "F.Cu") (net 3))
 (segment (start 130.125 66.775) (end 130.125 65.3269) (width 0.2) (layer "F.Cu") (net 3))
 (via (at 111.4761 70.8567) (size 0.6) (drill 0.3) (layers "F.Cu" "B.Cu") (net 3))
 (via (at 111.4761 88.9) (size 0.6) (drill 0.3) (layers "F.Cu" "B.Cu") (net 3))
 (segment (start 111.4761 88.9) (end 111.4761 70.8567) (width 0.2) (layer "B.Cu") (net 3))
 (segment (start 119.921 105.35) (end 107.5 105.35) (width 0.2) (layer "F.Cu") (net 2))
 (segment (start 120.071 105.5) (end 119.921 105.35) (width 0.2) (layer "F.Cu") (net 2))
 (segment (start 121.579 105.5) (end 120.071 105.5) (width 0.2) (layer "F.Cu") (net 2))
 (segment (start 129.621 69.4177) (end 134.38 69.4177) (width 0.2) (layer "F.Cu") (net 1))
 (segment (start 128.425 66.775) (end 128.425 68.2218) (width 0.2) (layer "F.Cu") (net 1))
 (segment (start 128.425 68.2218) (end 129.621 69.4177) (width 0.2) (layer "F.Cu") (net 1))
 (segment (start 134.38 105.5) (end 127.421 105.5) (width 0.2) (layer "F.Cu") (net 1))
 (via (at 134.38 69.4177) (size 0.6) (drill 0.3) (layers "F.Cu" "B.Cu") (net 1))
 (segment (start 134.38 105.5) (end 134.38 69.4177) (width 0.2) (layer "B.Cu") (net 1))
 (segment (start 149.323 70.7562) (end 143.756 70.7562) (width 0.2) (layer "F.Cu") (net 5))
 (segment (start 143.379 70.6211) (end 143.5 70.5) (width 0.2) (layer "F.Cu") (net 5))
 (segment (start 127.432 70.6211) (end 143.379 70.6211) (width 0.2) (layer "F.Cu") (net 5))
 (segment (start 125.025 68.2144) (end 127.432 70.6211) (width 0.2) (layer "F.Cu") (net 5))
 (segment (start 143.756 70.7562) (end 143.5 70.5) (width 0.2) (layer "F.Cu") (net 5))
 (segment (start 125.025 66.775) (end 125.025 68.2144) (width 0.2) (layer "F.Cu") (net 5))
 (via (at 149.323 70.7562) (size 0.6) (drill 0.3) (layers "F.Cu" "B.Cu") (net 5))
 (segment (start 149.323 76.0311) (end 149.323 70.7562) (width 0.2) (layer "B.Cu") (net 5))
 (segment (start 156 82.7083) (end 149.323 76.0311) (width 0.2) (layer "B.Cu") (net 5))
 (segment (start 156 84) (end 156 82.7083) (width 0.2) (layer "B.Cu") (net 5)))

